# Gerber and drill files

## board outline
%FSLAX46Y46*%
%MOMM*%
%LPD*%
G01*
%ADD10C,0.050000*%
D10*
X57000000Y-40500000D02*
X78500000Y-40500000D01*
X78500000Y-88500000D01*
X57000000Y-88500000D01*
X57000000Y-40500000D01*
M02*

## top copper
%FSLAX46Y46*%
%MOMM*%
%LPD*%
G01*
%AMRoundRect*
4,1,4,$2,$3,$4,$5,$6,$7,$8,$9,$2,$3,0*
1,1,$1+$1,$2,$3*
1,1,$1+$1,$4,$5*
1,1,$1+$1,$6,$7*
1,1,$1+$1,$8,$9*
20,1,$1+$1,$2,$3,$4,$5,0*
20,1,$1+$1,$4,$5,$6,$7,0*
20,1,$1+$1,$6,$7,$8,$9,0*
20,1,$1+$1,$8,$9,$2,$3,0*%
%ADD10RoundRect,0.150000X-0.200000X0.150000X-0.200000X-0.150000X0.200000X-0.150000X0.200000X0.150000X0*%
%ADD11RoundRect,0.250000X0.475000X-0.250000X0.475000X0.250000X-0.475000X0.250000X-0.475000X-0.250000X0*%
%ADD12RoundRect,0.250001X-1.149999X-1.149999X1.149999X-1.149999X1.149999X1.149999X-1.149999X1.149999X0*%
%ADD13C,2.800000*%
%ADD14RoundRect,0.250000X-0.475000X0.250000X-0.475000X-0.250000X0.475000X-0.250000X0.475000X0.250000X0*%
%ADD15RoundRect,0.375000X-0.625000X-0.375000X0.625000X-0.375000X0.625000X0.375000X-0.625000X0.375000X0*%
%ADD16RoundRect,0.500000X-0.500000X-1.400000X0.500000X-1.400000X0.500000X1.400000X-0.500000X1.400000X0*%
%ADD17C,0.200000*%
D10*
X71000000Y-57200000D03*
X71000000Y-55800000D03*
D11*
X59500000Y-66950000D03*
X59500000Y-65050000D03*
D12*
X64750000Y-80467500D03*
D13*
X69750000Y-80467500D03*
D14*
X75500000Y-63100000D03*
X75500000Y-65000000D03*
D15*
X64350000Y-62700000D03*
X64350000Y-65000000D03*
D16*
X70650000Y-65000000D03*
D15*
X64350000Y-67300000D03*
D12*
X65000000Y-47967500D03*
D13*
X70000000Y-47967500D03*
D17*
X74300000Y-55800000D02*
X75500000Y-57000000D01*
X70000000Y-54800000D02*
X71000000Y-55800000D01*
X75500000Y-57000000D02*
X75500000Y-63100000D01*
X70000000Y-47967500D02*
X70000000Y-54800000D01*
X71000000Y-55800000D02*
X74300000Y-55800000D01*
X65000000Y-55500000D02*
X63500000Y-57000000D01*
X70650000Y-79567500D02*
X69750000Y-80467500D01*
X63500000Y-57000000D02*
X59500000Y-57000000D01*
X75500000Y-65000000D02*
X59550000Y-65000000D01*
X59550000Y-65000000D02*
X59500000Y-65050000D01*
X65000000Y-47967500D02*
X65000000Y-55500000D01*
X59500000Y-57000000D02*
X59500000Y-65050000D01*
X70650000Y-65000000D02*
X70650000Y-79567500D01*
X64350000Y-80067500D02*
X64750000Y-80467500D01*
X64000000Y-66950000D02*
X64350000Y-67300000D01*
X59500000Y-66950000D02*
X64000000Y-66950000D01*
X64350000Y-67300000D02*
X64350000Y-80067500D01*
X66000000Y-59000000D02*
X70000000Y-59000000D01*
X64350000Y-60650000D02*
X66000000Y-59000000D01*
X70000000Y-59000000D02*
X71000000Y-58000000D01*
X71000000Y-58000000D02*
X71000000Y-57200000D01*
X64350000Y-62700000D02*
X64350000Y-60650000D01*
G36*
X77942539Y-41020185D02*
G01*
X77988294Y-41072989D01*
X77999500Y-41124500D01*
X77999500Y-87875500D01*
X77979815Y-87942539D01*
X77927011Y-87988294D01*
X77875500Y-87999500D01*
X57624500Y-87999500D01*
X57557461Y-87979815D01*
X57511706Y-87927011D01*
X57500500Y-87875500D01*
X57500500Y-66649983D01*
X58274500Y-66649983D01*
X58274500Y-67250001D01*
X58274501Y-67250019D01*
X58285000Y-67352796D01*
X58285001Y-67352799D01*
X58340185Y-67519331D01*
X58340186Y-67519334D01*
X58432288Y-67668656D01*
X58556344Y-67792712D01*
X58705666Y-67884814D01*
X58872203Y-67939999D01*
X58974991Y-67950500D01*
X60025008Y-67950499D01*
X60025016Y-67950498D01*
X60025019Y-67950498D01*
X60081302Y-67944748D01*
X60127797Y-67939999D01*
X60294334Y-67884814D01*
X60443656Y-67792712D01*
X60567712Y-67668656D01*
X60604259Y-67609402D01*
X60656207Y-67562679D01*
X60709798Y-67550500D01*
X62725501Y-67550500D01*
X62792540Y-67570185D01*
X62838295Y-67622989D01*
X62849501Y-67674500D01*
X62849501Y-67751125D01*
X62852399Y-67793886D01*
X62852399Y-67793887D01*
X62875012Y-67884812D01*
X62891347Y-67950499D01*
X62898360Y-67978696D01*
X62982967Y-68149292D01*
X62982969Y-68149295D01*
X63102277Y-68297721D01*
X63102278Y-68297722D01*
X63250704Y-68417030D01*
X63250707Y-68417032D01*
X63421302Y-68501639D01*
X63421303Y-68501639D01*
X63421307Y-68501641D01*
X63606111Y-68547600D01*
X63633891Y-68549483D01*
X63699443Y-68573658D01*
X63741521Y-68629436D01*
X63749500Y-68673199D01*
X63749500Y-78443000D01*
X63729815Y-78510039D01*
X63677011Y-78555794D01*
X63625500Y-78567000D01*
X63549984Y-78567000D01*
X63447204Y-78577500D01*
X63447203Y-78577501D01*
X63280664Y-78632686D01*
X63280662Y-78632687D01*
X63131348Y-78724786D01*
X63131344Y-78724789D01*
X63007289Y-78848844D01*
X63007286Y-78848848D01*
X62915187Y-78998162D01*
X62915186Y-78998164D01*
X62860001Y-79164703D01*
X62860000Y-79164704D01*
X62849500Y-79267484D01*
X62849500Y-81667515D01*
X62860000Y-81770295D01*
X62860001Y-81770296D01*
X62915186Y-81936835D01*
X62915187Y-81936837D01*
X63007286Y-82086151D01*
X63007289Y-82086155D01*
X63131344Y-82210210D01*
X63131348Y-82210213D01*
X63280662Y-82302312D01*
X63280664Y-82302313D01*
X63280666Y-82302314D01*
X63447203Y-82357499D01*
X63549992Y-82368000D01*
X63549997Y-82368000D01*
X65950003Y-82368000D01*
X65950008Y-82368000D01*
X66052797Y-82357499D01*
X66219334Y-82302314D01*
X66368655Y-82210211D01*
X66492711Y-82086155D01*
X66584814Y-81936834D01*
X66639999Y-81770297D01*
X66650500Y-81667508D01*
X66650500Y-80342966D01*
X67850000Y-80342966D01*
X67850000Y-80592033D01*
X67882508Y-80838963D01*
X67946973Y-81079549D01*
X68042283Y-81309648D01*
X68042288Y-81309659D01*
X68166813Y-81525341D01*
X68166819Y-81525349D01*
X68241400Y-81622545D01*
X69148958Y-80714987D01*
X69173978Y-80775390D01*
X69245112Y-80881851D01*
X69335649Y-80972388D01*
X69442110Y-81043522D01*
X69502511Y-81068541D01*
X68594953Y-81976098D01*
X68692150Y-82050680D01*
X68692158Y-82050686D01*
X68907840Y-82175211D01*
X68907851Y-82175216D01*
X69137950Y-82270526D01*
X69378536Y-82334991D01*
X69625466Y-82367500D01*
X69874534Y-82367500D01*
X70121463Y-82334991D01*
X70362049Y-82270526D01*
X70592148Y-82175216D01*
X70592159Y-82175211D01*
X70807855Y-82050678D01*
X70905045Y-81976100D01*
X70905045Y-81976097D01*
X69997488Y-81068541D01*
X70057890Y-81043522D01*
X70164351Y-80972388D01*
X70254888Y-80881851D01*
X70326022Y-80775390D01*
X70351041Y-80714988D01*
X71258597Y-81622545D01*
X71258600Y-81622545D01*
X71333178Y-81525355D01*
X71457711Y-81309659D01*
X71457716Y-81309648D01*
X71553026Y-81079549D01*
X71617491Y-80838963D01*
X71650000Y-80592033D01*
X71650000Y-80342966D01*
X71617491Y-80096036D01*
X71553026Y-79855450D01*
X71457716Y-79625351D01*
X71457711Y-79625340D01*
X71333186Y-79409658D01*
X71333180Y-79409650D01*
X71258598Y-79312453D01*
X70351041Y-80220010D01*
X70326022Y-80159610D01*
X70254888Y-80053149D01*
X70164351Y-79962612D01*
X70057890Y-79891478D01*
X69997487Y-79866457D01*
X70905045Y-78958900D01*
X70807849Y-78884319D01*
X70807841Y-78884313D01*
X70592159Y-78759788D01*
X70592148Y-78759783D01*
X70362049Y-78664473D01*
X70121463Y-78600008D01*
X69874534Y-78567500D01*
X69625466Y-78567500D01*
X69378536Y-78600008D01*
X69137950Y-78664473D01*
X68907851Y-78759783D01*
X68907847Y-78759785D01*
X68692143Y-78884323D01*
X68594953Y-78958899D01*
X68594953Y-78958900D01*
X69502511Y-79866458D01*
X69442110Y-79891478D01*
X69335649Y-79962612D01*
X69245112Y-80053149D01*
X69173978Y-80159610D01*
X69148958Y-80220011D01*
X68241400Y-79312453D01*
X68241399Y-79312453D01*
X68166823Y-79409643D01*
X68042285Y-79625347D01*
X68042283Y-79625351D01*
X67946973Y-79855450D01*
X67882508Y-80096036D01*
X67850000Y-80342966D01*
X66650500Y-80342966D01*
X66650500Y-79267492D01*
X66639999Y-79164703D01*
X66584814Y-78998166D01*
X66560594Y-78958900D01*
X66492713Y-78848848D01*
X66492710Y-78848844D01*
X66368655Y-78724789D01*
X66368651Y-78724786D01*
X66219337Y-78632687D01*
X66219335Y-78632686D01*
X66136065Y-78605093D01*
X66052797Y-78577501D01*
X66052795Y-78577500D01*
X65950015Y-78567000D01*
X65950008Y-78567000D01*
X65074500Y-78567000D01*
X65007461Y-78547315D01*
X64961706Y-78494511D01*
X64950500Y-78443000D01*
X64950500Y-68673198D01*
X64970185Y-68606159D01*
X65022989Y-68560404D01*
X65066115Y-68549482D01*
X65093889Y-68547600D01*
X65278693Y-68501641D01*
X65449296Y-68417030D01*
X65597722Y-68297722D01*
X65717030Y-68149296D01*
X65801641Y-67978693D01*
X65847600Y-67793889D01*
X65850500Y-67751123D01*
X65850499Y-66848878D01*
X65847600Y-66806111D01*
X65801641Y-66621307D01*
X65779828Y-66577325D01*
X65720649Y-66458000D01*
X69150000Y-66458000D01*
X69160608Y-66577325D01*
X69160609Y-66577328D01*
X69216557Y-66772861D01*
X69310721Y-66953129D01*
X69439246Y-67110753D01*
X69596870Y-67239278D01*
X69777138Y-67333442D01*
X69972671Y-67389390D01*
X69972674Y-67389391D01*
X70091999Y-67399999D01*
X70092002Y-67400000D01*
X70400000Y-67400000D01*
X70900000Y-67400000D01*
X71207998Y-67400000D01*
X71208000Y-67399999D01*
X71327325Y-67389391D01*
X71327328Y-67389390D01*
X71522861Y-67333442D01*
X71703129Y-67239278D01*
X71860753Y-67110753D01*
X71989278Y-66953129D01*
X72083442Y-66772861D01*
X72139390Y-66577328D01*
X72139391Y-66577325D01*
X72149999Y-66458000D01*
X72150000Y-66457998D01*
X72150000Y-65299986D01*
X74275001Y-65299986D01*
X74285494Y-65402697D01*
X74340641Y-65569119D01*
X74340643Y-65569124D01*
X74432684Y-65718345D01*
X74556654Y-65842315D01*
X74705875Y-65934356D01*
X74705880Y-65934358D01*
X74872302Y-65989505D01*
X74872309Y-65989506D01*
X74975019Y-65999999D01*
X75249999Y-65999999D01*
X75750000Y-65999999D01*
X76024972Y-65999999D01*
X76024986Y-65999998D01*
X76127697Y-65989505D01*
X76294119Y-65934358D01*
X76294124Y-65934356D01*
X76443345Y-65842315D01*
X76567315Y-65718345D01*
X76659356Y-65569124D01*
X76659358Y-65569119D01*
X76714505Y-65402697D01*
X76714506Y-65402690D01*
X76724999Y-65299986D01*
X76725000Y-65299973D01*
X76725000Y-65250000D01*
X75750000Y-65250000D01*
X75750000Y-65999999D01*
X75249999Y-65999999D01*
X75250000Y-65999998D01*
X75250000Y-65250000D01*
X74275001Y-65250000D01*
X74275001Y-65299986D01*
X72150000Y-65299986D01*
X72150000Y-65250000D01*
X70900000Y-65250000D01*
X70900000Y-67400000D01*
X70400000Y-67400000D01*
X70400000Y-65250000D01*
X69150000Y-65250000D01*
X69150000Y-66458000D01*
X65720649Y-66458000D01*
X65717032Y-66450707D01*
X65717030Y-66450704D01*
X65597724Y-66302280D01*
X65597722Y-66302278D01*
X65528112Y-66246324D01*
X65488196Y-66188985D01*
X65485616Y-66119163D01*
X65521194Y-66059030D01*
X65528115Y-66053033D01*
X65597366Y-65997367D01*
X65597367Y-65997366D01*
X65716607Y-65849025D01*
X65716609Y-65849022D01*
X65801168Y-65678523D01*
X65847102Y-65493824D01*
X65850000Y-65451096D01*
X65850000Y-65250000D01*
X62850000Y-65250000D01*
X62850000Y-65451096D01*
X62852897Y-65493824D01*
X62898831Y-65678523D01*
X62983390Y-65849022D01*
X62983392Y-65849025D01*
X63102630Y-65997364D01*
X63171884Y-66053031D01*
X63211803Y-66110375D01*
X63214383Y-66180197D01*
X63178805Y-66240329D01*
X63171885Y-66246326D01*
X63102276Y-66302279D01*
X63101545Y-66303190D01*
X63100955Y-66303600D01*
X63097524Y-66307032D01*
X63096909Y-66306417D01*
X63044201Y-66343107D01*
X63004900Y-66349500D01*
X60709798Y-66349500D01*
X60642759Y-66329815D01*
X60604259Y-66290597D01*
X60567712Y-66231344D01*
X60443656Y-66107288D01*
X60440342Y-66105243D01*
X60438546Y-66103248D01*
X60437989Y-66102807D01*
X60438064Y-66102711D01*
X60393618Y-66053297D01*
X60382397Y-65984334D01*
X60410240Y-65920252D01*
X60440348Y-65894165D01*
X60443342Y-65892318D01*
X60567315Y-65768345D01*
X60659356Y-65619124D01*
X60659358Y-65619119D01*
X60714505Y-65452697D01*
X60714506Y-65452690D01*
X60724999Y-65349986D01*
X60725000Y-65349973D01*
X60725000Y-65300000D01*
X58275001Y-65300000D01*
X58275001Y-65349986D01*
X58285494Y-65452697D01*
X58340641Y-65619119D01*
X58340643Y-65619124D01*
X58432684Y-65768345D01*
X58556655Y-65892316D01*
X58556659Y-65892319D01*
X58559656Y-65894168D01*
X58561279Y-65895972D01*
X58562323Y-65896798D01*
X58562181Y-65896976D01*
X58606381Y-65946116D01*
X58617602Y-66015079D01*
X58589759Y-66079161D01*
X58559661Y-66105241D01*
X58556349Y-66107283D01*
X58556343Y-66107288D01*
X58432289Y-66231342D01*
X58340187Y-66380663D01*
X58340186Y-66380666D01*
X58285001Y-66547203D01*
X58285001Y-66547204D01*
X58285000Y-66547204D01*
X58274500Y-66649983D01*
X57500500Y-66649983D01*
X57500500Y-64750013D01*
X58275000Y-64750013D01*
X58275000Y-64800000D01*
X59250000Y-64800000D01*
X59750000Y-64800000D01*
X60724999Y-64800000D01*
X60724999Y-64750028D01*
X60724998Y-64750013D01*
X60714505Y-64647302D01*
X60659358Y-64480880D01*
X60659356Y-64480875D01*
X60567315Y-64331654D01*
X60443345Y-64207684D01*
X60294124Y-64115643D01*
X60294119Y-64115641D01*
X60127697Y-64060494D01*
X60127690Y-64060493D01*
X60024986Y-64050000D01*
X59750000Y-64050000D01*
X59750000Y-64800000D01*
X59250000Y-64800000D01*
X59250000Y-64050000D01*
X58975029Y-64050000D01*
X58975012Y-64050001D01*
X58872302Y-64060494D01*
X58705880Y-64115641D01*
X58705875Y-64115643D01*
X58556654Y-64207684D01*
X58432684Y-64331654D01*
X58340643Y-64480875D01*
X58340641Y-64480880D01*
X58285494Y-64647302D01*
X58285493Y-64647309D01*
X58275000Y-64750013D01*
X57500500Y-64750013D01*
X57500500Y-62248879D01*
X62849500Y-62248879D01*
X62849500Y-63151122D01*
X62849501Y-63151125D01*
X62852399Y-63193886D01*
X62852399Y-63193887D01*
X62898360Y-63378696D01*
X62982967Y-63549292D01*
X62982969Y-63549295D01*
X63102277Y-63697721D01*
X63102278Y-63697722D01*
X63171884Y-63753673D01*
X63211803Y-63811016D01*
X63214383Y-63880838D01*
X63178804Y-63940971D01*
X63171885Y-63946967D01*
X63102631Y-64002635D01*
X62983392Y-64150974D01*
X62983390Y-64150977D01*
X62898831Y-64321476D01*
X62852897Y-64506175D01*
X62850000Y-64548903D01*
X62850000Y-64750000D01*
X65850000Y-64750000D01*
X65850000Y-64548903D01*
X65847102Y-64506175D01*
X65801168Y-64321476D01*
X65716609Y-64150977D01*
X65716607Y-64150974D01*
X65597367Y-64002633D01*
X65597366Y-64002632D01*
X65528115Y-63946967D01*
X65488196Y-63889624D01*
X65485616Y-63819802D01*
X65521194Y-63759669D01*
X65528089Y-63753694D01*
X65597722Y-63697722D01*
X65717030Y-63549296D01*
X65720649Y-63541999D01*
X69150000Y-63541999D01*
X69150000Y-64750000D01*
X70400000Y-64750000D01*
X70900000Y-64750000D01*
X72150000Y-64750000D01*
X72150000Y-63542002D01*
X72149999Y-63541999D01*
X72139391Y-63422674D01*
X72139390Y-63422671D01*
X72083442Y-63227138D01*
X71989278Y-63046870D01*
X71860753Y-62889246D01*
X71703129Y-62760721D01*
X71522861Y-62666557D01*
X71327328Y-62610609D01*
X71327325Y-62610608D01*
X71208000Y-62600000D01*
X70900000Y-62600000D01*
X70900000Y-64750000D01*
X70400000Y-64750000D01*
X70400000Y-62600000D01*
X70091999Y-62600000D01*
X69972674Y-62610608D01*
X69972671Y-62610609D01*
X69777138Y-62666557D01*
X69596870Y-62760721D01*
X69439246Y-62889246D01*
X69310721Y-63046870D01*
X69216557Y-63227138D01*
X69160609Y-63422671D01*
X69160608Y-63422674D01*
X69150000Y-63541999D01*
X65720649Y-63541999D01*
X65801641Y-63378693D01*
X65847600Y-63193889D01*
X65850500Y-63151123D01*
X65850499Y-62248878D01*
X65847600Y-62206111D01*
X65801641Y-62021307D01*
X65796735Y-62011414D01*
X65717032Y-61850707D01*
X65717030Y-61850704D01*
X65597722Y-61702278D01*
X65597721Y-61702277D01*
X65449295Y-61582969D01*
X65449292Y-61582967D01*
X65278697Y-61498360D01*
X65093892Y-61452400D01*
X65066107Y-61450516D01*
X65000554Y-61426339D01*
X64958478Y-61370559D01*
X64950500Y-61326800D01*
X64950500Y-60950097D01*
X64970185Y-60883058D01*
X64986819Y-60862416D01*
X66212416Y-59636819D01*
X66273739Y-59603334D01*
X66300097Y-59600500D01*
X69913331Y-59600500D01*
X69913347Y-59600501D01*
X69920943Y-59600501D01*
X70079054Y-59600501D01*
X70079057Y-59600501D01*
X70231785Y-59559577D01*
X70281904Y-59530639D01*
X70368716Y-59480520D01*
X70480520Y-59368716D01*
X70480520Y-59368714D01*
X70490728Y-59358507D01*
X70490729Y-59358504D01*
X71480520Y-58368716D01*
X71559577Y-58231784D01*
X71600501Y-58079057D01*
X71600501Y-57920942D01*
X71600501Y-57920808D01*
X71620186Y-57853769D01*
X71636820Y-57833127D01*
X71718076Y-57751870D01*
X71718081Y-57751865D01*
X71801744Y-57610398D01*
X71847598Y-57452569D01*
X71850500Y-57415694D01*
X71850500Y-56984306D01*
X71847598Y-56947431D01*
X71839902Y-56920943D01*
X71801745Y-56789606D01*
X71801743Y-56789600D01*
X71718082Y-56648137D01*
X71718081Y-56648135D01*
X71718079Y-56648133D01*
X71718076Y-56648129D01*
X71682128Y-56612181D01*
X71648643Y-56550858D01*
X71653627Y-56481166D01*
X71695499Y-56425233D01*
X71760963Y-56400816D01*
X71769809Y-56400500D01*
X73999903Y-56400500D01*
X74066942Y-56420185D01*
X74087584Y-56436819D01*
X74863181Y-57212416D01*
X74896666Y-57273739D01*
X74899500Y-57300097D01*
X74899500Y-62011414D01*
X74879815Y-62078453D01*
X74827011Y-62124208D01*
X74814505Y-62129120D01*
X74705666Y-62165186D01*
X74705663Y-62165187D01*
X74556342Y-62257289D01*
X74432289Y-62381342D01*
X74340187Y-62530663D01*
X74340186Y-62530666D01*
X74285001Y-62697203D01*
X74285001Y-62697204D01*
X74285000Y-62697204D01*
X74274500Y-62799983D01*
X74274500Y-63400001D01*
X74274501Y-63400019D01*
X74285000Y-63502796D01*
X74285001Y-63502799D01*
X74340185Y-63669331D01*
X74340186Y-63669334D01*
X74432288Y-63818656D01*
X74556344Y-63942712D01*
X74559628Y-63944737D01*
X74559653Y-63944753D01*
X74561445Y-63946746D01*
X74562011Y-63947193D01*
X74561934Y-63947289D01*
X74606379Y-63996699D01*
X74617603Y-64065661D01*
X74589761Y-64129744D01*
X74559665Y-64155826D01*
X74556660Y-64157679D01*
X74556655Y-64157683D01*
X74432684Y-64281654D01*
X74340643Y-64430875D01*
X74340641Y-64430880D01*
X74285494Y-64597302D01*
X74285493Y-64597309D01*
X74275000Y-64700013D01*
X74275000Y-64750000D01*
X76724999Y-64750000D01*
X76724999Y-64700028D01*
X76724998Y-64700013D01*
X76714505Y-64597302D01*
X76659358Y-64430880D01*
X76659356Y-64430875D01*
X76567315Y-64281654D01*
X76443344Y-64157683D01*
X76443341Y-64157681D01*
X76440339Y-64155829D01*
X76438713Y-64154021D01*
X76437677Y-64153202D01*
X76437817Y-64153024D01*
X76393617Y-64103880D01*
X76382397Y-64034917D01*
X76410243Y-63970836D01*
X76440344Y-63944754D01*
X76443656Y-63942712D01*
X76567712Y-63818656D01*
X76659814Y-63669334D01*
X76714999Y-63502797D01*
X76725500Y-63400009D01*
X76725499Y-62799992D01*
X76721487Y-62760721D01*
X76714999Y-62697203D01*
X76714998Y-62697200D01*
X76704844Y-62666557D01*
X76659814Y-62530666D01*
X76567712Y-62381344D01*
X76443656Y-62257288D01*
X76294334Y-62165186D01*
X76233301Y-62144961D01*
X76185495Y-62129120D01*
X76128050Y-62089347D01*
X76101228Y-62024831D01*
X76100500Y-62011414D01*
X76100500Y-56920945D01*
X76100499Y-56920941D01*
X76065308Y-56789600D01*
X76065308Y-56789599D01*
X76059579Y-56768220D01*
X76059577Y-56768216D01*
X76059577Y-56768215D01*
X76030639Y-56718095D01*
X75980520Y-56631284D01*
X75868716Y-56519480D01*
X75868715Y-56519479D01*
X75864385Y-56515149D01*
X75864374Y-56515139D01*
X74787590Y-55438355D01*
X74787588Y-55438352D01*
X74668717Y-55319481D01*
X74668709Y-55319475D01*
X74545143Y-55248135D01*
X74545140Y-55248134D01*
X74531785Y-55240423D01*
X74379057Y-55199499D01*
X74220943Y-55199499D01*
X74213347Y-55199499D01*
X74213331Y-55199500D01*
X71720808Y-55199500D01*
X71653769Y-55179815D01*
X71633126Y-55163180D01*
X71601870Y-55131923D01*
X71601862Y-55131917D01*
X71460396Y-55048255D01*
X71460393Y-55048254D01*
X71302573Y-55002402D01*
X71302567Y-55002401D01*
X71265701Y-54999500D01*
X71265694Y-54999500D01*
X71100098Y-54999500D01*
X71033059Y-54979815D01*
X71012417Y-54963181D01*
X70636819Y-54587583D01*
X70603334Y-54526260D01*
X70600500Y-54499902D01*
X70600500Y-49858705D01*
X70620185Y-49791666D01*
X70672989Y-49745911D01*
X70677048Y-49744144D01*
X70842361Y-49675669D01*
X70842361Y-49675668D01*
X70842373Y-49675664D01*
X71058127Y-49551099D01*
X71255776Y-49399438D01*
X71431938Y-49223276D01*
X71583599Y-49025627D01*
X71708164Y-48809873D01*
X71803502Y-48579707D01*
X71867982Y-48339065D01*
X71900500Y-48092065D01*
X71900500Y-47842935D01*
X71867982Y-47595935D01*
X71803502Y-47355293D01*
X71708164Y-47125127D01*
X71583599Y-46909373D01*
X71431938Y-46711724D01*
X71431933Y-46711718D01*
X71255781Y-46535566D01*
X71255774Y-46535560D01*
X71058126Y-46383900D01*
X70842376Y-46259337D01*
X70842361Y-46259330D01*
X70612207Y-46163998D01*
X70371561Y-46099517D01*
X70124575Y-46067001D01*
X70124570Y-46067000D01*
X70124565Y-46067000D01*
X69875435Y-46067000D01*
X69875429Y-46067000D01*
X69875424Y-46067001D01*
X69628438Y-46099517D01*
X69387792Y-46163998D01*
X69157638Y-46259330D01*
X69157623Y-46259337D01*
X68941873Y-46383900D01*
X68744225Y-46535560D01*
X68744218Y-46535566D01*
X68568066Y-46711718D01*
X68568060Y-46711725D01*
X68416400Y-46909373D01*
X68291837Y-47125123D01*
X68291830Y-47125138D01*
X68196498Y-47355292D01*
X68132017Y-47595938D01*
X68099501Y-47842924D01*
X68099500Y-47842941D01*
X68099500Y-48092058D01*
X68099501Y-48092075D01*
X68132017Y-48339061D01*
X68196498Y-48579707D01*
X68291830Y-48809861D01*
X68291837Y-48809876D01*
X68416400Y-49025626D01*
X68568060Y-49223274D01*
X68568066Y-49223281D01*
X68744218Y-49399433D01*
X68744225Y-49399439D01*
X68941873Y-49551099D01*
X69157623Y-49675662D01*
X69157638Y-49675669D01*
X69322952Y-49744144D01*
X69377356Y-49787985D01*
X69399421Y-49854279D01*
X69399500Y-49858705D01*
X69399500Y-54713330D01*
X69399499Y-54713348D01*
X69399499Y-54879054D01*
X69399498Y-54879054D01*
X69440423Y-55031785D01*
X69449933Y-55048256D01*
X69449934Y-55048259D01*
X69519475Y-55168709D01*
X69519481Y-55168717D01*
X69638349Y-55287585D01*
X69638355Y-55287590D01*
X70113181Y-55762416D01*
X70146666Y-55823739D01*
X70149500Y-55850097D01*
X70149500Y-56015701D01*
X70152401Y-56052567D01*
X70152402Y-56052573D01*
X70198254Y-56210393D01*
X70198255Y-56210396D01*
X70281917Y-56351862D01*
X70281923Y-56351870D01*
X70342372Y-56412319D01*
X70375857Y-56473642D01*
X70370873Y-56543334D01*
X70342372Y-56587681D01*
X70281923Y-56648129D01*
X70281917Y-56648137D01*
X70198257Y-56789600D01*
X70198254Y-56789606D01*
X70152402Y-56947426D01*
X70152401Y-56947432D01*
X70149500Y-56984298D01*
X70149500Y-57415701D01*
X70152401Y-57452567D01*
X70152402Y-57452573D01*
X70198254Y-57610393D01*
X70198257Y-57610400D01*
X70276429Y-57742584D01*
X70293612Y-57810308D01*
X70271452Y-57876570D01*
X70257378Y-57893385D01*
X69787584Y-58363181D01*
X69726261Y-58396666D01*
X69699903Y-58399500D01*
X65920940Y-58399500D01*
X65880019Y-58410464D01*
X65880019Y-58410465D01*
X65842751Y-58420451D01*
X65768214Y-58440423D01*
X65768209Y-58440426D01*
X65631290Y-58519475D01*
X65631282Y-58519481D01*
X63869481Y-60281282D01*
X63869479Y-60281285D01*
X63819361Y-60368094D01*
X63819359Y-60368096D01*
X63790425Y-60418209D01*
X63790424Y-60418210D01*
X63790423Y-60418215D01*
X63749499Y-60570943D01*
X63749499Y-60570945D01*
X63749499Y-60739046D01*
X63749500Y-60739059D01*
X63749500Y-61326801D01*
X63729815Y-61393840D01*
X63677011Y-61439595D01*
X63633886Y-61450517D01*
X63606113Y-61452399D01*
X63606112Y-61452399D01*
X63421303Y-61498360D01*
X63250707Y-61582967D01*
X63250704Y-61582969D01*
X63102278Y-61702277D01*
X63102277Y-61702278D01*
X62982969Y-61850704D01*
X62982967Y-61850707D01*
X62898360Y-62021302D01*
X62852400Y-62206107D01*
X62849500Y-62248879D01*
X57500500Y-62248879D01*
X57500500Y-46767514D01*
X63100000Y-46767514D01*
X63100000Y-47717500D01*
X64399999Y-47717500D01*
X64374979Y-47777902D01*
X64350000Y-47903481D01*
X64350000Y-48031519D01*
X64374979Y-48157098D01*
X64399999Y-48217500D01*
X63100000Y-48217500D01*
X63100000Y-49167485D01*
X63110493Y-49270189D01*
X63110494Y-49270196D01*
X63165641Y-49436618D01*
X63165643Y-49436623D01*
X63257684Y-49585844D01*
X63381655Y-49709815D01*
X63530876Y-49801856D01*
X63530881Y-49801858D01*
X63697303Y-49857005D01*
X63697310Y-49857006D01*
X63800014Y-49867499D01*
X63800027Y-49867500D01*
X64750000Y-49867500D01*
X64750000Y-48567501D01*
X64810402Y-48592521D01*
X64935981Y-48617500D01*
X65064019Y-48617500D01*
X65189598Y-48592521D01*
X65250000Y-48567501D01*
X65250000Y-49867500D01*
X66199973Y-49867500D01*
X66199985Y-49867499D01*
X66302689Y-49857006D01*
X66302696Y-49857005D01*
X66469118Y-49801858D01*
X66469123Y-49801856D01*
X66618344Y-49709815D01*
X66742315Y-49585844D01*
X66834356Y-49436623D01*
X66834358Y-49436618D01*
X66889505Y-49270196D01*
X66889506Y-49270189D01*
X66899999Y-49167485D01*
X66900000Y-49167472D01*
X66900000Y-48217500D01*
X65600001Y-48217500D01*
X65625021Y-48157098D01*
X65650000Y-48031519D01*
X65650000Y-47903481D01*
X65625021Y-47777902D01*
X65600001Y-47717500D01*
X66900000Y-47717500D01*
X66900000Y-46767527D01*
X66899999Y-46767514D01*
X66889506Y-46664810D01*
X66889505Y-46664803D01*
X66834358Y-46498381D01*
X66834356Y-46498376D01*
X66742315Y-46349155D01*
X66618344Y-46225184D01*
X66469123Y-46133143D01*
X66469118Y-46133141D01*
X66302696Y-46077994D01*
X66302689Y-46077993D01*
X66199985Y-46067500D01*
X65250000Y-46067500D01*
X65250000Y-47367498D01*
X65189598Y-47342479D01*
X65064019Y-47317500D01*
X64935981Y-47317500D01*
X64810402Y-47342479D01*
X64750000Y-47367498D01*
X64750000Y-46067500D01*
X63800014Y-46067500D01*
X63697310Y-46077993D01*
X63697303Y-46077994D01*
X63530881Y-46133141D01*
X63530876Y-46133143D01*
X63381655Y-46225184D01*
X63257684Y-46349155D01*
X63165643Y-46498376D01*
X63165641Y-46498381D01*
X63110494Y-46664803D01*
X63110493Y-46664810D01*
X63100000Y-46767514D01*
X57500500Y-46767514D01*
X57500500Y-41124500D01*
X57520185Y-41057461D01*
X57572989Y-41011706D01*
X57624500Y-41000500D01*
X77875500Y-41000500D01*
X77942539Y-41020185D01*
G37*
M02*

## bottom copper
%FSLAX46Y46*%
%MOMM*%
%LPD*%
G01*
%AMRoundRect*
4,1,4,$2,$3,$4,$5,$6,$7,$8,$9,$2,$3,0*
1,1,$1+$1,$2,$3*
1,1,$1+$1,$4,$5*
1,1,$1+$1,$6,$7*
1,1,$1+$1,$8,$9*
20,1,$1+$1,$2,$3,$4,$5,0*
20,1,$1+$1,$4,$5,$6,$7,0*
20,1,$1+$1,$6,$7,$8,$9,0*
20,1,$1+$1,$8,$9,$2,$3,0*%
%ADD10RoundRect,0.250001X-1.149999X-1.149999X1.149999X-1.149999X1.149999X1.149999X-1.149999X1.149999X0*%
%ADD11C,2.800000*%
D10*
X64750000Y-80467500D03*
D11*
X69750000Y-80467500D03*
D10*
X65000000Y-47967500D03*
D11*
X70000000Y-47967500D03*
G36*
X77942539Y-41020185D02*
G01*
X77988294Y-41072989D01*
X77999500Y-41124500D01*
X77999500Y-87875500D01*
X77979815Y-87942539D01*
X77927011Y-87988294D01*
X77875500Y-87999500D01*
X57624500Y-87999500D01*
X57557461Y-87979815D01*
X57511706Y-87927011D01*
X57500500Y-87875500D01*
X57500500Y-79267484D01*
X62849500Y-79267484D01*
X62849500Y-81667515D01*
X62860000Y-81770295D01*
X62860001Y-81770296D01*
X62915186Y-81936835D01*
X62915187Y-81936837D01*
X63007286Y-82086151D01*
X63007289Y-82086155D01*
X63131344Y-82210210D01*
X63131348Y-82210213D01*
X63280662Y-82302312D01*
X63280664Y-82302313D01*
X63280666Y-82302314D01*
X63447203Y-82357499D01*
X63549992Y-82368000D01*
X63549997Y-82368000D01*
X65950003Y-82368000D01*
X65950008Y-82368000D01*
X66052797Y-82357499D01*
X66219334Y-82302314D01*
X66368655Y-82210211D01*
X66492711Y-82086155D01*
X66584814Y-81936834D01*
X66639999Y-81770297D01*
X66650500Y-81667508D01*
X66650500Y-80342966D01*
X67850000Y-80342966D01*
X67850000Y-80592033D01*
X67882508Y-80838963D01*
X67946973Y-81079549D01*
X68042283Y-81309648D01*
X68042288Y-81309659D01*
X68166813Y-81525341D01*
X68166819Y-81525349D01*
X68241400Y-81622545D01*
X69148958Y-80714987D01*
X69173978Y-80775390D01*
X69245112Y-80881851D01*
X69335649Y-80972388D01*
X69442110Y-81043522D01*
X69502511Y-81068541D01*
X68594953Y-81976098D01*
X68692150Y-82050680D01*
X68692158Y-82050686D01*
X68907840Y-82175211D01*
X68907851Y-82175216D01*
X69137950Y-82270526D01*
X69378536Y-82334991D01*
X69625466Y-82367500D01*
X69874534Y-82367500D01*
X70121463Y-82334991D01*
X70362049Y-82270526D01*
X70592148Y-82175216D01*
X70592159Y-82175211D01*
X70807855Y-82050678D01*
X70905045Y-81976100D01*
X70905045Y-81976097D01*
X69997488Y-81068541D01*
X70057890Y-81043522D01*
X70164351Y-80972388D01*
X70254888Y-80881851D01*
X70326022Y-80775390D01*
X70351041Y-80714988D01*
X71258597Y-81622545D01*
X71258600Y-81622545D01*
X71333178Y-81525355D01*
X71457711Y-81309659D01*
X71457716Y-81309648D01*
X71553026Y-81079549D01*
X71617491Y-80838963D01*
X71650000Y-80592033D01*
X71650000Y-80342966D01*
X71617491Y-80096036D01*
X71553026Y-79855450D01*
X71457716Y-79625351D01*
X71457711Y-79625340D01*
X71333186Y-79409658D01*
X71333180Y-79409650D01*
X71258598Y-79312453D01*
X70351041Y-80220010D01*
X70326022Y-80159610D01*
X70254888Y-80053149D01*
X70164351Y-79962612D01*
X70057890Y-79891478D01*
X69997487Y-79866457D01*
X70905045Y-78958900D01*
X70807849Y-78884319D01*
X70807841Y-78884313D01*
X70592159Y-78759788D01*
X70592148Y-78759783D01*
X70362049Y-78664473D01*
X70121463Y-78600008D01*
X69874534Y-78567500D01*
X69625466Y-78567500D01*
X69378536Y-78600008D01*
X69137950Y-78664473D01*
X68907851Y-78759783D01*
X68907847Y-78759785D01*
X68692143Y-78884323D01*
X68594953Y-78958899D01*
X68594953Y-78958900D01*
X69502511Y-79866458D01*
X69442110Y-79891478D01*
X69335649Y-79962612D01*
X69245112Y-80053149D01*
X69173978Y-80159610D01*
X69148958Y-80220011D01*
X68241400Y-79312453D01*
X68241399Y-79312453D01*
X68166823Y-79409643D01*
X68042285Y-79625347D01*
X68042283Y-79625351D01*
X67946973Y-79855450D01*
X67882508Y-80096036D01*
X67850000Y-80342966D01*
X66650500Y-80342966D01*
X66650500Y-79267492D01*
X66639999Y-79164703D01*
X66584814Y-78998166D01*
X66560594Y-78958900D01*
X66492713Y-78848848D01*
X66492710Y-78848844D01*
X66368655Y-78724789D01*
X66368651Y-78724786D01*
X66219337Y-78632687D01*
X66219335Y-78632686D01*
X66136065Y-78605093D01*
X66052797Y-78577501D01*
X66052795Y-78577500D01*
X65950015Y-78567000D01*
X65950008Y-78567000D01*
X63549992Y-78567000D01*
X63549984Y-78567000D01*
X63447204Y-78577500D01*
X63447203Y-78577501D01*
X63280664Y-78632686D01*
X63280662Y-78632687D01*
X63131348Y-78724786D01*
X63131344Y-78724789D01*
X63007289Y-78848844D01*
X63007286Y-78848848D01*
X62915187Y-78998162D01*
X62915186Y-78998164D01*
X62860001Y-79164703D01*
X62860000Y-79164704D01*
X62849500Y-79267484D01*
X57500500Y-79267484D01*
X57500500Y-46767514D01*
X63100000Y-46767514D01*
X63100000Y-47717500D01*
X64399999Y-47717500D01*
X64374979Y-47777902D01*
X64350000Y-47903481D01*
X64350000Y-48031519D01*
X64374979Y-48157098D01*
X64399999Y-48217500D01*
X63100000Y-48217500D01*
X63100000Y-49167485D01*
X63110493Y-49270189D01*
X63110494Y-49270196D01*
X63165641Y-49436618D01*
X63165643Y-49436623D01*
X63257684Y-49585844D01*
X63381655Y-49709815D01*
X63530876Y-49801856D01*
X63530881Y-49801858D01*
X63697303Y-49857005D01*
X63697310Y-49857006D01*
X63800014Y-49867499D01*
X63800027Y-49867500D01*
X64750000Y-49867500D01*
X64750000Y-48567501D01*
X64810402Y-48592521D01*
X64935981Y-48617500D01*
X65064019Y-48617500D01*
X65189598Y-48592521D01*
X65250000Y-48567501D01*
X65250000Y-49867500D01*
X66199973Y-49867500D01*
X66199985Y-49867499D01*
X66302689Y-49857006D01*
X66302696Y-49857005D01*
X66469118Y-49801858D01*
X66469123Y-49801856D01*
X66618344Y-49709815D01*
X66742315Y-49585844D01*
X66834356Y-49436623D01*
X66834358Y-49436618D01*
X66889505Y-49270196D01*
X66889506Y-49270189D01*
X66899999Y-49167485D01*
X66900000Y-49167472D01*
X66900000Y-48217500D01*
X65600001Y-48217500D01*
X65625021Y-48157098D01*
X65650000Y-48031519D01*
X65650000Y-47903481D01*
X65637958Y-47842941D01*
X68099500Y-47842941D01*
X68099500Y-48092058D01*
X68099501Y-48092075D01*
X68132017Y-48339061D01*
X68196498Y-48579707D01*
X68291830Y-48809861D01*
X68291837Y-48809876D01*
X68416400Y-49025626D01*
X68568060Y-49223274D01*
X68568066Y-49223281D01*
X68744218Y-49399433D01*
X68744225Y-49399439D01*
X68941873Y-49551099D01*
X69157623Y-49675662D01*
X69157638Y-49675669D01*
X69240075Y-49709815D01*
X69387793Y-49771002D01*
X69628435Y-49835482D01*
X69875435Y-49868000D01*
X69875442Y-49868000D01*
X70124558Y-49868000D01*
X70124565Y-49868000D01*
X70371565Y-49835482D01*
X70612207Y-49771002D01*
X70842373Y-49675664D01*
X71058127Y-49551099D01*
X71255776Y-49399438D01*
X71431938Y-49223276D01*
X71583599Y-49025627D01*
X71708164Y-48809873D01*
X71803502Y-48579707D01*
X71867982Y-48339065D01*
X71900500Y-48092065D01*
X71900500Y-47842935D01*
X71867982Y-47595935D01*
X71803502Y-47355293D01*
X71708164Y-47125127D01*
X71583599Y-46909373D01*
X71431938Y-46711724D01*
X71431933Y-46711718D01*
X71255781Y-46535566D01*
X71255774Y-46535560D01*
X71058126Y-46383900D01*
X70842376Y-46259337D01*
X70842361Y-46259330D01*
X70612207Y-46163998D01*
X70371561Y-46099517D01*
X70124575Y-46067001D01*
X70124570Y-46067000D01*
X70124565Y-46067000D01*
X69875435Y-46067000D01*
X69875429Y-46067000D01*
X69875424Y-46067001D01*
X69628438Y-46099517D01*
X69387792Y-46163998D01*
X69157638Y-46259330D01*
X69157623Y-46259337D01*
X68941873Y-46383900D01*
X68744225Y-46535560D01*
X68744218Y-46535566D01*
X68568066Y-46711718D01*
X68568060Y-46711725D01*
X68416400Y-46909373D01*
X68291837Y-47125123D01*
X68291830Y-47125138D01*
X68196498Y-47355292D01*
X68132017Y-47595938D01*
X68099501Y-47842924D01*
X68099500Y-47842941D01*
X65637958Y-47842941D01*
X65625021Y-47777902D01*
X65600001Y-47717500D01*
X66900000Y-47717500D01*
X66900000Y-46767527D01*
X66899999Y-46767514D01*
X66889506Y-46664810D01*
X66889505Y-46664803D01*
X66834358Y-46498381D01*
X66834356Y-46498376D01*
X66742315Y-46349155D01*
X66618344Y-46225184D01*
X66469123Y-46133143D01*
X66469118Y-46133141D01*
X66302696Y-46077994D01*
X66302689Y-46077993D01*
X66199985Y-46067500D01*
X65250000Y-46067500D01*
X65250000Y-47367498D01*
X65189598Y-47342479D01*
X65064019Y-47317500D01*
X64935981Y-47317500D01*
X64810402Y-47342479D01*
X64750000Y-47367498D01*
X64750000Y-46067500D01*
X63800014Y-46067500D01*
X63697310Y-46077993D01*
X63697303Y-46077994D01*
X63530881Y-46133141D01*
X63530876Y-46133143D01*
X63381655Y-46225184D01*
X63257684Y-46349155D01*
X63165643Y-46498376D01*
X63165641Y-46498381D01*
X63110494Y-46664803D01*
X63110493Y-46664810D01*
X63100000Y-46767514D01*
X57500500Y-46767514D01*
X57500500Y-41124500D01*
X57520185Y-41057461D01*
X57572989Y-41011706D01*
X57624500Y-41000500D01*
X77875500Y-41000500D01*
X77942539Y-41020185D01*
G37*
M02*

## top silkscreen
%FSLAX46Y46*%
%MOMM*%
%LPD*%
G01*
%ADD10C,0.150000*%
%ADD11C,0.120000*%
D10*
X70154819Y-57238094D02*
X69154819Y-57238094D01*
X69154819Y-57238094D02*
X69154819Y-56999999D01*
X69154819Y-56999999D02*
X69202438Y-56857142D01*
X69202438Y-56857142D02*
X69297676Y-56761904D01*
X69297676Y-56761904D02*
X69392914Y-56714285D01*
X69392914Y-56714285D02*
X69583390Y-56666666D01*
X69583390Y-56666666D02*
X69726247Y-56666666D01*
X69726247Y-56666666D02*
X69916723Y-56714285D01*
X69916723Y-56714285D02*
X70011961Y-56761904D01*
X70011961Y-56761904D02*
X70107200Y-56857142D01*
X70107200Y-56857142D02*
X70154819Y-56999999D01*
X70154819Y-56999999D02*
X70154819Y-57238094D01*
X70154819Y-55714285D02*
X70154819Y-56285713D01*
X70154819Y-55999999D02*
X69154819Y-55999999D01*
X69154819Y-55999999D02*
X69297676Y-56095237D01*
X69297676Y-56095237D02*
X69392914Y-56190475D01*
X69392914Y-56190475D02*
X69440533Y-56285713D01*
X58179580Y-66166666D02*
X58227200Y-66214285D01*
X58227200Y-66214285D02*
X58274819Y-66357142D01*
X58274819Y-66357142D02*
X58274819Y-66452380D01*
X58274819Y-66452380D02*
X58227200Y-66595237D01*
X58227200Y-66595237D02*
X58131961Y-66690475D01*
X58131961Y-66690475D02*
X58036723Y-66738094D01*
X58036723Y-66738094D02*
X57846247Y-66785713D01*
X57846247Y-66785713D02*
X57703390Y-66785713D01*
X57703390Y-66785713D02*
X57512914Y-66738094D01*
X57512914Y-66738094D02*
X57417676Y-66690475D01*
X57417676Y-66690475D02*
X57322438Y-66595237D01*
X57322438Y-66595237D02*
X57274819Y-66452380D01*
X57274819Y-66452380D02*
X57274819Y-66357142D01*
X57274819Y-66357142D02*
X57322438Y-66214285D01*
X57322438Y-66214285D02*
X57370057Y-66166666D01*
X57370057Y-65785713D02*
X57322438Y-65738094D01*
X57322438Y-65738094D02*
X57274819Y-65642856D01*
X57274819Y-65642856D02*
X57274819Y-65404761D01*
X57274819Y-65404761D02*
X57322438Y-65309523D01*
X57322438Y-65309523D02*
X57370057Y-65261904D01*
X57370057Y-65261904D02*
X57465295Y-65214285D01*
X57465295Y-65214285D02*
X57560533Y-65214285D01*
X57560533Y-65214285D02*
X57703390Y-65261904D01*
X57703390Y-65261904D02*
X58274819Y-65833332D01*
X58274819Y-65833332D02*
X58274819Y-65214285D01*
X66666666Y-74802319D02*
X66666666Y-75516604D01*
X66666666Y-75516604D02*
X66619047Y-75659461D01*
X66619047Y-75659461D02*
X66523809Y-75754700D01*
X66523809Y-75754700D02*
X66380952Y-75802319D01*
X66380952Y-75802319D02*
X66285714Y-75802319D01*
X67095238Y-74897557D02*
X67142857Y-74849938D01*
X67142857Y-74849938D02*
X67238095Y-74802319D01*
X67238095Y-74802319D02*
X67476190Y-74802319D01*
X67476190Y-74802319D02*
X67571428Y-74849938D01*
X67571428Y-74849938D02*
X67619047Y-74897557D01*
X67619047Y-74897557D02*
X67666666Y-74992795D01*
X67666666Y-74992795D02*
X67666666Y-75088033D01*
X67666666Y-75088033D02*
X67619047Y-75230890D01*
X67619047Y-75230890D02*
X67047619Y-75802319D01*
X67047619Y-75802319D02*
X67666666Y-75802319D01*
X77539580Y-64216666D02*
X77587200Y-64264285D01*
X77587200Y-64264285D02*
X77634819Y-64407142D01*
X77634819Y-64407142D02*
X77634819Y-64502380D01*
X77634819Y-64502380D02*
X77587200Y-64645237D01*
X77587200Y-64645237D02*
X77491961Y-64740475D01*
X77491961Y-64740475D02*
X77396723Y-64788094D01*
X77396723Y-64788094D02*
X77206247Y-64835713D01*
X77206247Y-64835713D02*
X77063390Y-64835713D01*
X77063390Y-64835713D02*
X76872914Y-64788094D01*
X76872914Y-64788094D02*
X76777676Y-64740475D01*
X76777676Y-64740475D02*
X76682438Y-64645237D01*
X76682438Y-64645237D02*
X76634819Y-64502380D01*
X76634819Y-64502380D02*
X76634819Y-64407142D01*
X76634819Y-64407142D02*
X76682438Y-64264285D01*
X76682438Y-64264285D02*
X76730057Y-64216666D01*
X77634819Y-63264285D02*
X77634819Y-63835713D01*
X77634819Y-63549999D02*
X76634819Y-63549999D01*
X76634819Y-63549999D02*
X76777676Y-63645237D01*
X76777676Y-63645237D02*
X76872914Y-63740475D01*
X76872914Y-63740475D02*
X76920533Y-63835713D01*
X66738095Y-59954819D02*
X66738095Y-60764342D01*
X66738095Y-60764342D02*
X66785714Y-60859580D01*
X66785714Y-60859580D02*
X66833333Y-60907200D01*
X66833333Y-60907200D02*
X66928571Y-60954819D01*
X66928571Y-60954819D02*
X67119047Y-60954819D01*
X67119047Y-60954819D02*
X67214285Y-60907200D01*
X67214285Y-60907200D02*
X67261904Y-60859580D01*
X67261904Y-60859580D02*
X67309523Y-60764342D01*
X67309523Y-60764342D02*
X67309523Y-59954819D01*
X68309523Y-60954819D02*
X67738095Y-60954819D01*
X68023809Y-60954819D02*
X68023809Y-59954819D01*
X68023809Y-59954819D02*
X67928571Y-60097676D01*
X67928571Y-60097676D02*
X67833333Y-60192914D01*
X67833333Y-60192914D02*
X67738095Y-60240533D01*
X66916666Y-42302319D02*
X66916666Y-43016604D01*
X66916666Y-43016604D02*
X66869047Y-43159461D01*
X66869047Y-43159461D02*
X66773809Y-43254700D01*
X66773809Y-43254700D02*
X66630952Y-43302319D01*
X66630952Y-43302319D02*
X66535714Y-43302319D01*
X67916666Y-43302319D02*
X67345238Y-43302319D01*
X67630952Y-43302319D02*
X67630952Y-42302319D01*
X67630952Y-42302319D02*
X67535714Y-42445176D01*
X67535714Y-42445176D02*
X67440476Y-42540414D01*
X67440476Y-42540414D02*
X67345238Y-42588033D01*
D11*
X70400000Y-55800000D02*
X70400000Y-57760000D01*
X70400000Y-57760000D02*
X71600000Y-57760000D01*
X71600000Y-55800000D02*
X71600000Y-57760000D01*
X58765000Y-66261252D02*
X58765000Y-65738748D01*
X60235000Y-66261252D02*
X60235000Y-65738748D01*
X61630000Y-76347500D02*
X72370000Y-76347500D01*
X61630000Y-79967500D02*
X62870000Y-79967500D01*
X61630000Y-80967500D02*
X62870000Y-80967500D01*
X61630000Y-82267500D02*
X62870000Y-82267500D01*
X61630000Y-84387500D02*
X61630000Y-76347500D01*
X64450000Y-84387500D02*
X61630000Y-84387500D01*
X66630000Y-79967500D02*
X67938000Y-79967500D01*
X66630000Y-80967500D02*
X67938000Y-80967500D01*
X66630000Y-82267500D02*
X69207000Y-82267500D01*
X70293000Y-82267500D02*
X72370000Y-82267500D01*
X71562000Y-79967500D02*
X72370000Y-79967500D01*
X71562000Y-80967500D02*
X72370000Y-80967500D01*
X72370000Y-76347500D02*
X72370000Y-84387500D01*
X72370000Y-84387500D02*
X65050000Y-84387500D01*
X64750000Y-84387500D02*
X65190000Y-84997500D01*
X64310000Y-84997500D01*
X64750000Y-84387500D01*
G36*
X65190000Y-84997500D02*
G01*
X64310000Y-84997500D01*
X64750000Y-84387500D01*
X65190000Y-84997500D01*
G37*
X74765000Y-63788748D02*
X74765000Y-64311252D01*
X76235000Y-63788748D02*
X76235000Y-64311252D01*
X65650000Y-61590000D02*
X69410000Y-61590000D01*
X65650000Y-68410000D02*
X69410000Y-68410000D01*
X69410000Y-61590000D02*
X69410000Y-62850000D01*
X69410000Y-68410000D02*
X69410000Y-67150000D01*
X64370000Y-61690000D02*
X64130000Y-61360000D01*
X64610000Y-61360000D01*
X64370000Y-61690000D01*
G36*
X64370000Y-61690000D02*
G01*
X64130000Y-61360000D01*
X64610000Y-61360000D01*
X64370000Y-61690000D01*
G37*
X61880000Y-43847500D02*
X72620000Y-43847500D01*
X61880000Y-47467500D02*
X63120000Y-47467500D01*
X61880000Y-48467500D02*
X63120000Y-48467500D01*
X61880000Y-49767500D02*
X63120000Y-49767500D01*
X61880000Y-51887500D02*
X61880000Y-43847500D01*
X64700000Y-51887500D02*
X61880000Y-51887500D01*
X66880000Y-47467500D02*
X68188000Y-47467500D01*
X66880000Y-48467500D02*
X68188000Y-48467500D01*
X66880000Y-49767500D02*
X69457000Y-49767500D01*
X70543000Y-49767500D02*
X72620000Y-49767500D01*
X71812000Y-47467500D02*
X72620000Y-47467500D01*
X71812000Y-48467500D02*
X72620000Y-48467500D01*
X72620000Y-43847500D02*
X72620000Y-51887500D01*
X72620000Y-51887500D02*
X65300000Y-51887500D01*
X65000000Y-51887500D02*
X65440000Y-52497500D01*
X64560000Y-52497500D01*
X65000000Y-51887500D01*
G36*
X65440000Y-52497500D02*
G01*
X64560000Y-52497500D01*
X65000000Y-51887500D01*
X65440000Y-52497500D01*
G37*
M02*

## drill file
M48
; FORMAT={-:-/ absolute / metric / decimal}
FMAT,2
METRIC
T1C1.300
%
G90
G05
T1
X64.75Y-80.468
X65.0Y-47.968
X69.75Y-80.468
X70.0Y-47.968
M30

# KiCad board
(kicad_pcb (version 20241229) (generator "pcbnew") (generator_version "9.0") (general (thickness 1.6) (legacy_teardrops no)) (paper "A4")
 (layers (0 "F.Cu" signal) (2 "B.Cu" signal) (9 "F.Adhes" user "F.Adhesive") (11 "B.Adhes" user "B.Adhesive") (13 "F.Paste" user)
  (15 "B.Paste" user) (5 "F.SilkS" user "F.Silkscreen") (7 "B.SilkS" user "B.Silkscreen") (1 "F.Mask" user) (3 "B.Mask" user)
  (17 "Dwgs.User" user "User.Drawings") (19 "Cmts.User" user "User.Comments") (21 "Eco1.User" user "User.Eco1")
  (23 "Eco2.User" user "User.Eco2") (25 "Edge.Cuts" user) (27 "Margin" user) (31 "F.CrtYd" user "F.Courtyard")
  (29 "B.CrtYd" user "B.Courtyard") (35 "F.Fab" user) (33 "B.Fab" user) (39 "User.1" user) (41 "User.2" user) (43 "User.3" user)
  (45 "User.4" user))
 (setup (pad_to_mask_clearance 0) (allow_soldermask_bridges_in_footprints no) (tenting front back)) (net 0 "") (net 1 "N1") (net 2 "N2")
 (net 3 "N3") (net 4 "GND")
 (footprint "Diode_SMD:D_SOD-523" (layer "F.Cu") (at 71 56.5 90)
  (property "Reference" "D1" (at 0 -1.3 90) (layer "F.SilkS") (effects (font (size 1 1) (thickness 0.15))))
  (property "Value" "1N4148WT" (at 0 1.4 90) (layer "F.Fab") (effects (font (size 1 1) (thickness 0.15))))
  (fp_line (start 0.7 -0.6) (end -1.26 -0.6) (stroke (width 0.12) (type solid)) (layer "F.SilkS"))
  (fp_line (start -1.26 -0.6) (end -1.26 0.6) (stroke (width 0.12) (type solid)) (layer "F.SilkS"))
  (fp_line (start 0.7 0.6) (end -1.26 0.6) (stroke (width 0.12) (type solid)) (layer "F.SilkS"))
  (pad "1" smd roundrect (at -0.7 0 270) (size 0.6 0.7) (layers "F.Cu" "F.Mask" "F.Paste") (roundrect_rratio 0.25) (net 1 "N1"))
  (pad "2" smd roundrect (at 0.7 0 270) (size 0.6 0.7) (layers "F.Cu" "F.Mask" "F.Paste") (roundrect_rratio 0.25) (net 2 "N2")))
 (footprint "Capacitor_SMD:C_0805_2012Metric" (layer "F.Cu") (at 59.5 66 90)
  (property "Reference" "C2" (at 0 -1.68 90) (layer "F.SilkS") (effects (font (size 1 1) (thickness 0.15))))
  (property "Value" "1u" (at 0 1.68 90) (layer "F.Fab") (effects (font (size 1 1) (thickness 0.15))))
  (fp_line (start -0.261252 -0.735) (end 0.261252 -0.735) (stroke (width 0.12) (type solid)) (layer "F.SilkS"))
  (fp_line (start -0.261252 0.735) (end 0.261252 0.735) (stroke (width 0.12) (type solid)) (layer "F.SilkS"))
  (pad "1" smd roundrect (at -0.95 0 90) (size 1 1.45) (layers "F.Cu" "F.Mask" "F.Paste") (roundrect_rratio 0.25) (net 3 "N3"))
  (pad "2" smd roundrect (at 0.95 0 90) (size 1 1.45) (layers "F.Cu" "F.Mask" "F.Paste") (roundrect_rratio 0.25) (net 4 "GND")))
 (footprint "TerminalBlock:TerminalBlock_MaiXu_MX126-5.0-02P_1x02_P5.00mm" (layer "F.Cu") (at 64.75 80.4675)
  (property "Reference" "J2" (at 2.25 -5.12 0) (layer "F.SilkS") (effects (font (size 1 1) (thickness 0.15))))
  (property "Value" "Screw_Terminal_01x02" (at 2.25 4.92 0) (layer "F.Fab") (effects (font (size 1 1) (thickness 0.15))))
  (fp_line (start -3.12 -4.12) (end 7.62 -4.12) (stroke (width 0.12) (type solid)) (layer "F.SilkS"))
  (fp_line (start -3.12 -0.5) (end -1.88 -0.5) (stroke (width 0.12) (type solid)) (layer "F.SilkS"))
  (fp_line (start -3.12 0.5) (end -1.88 0.5) (stroke (width 0.12) (type solid)) (layer "F.SilkS"))
  (fp_line (start -3.12 1.8) (end -1.88 1.8) (stroke (width 0.12) (type solid)) (layer "F.SilkS"))
  (fp_line (start -3.12 3.92) (end -3.12 -4.12) (stroke (width 0.12) (type solid)) (layer "F.SilkS"))
  (fp_line (start -0.3 3.92) (end -3.12 3.92) (stroke (width 0.12) (type solid)) (layer "F.SilkS"))
  (fp_line (start 1.88 -0.5) (end 3.188 -0.5) (stroke (width 0.12) (type solid)) (layer "F.SilkS"))
  (fp_line (start 1.88 0.5) (end 3.188 0.5) (stroke (width 0.12) (type solid)) (layer "F.SilkS"))
  (fp_line (start 1.88 1.8) (end 4.457 1.8) (stroke (width 0.12) (type solid)) (layer "F.SilkS"))
  (fp_line (start 5.543 1.8) (end 7.62 1.8) (stroke (width 0.12) (type solid)) (layer "F.SilkS"))
  (fp_line (start 6.812 -0.5) (end 7.62 -0.5) (stroke (width 0.12) (type solid)) (layer "F.SilkS"))
  (fp_line (start 6.812 0.5) (end 7.62 0.5) (stroke (width 0.12) (type solid)) (layer "F.SilkS"))
  (fp_line (start 7.62 -4.12) (end 7.62 3.92) (stroke (width 0.12) (type solid)) (layer "F.SilkS"))
  (fp_line (start 7.62 3.92) (end 0.3 3.92) (stroke (width 0.12) (type solid)) (layer "F.SilkS"))
  (fp_poly (pts (xy 0 3.92) (xy 0.44 4.53) (xy -0.44 4.53)) (stroke (width 0.12) (type solid)) (fill yes) (layer "F.SilkS"))
  (pad "1" thru_hole roundrect (at 0 0) (size 2.8 2.8) (drill 1.3) (layers "*.Cu" "*.Mask") (remove_unused_layers no)
   (roundrect_rratio 0.089286) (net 3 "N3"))
  (pad "2" thru_hole circle (at 5 0) (size 2.8 2.8) (drill 1.3) (layers "*.Cu" "*.Mask") (remove_unused_layers no) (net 4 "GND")))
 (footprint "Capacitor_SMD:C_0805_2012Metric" (layer "F.Cu") (at 75.5 64.05 -90)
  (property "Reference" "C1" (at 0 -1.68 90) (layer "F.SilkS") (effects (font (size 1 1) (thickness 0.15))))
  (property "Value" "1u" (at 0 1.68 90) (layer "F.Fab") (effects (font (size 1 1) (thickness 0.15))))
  (fp_line (start -0.261252 0.735) (end 0.261252 0.735) (stroke (width 0.12) (type solid)) (layer "F.SilkS"))
  (fp_line (start -0.261252 -0.735) (end 0.261252 -0.735) (stroke (width 0.12) (type solid)) (layer "F.SilkS"))
  (pad "1" smd roundrect (at -0.95 0 270) (size 1 1.45) (layers "F.Cu" "F.Mask" "F.Paste") (roundrect_rratio 0.25) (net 2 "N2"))
  (pad "2" smd roundrect (at 0.95 0 270) (size 1 1.45) (layers "F.Cu" "F.Mask" "F.Paste") (roundrect_rratio 0.25) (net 4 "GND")))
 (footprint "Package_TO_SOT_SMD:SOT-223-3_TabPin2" (layer "F.Cu") (at 67.5 65)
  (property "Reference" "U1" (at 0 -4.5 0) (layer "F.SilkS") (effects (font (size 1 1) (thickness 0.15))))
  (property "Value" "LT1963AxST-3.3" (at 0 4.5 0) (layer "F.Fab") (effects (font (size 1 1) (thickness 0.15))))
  (fp_line (start -1.85 -3.41) (end 1.91 -3.41) (stroke (width 0.12) (type solid)) (layer "F.SilkS"))
  (fp_line (start -1.85 3.41) (end 1.91 3.41) (stroke (width 0.12) (type solid)) (layer "F.SilkS"))
  (fp_line (start 1.91 -3.41) (end 1.91 -2.15) (stroke (width 0.12) (type solid)) (layer "F.SilkS"))
  (fp_line (start 1.91 3.41) (end 1.91 2.15) (stroke (width 0.12) (type solid)) (layer "F.SilkS"))
  (fp_poly
   (pts (xy -3.13 -3.31) (xy -3.37 -3.64) (xy -2.89 -3.64) (xy -3.13 -3.31)) (stroke (width 0.12) (type solid)) (fill yes) (layer "F.SilkS"))
  (pad "1" smd roundrect (at -3.15 -2.3) (size 2 1.5) (layers "F.Cu" "F.Mask" "F.Paste") (roundrect_rratio 0.25) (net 1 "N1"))
  (pad "2" smd roundrect (at -3.15 0) (size 2 1.5) (layers "F.Cu" "F.Mask" "F.Paste") (roundrect_rratio 0.25) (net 4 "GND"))
  (pad "2" smd roundrect (at 3.15 0) (size 2 3.8) (layers "F.Cu" "F.Mask" "F.Paste") (roundrect_rratio 0.25) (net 4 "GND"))
  (pad "3" smd roundrect (at -3.15 2.3) (size 2 1.5) (layers "F.Cu" "F.Mask" "F.Paste") (roundrect_rratio 0.25) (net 3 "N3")))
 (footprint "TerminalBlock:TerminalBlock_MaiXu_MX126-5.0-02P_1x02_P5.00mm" (layer "F.Cu") (at 65 47.9675)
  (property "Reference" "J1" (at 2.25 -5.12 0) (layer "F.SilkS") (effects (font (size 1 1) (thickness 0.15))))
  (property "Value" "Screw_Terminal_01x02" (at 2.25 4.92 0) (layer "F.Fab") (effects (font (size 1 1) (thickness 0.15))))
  (fp_line (start -3.12 -4.12) (end 7.62 -4.12) (stroke (width 0.12) (type solid)) (layer "F.SilkS"))
  (fp_line (start -3.12 -0.5) (end -1.88 -0.5) (stroke (width 0.12) (type solid)) (layer "F.SilkS"))
  (fp_line (start -3.12 0.5) (end -1.88 0.5) (stroke (width 0.12) (type solid)) (layer "F.SilkS"))
  (fp_line (start -3.12 1.8) (end -1.88 1.8) (stroke (width 0.12) (type solid)) (layer "F.SilkS"))
  (fp_line (start -3.12 3.92) (end -3.12 -4.12) (stroke (width 0.12) (type solid)) (layer "F.SilkS"))
  (fp_line (start -0.3 3.92) (end -3.12 3.92) (stroke (width 0.12) (type solid)) (layer "F.SilkS"))
  (fp_line (start 1.88 -0.5) (end 3.188 -0.5) (stroke (width 0.12) (type solid)) (layer "F.SilkS"))
  (fp_line (start 1.88 0.5) (end 3.188 0.5) (stroke (width 0.12) (type solid)) (layer "F.SilkS"))
  (fp_line (start 1.88 1.8) (end 4.457 1.8) (stroke (width 0.12) (type solid)) (layer "F.SilkS"))
  (fp_line (start 5.543 1.8) (end 7.62 1.8) (stroke (width 0.12) (type solid)) (layer "F.SilkS"))
  (fp_line (start 6.812 -0.5) (end 7.62 -0.5) (stroke (width 0.12) (type solid)) (layer "F.SilkS"))
  (fp_line (start 6.812 0.5) (end 7.62 0.5) (stroke (width 0.12) (type solid)) (layer "F.SilkS"))
  (fp_line (start 7.62 -4.12) (end 7.62 3.92) (stroke (width 0.12) (type solid)) (layer "F.SilkS"))
  (fp_line (start 7.62 3.92) (end 0.3 3.92) (stroke (width 0.12) (type solid)) (layer "F.SilkS"))
  (fp_poly (pts (xy 0 3.92) (xy 0.44 4.53) (xy -0.44 4.53)) (stroke (width 0.12) (type solid)) (fill yes) (layer "F.SilkS"))
  (pad "1" thru_hole roundrect (at 0 0) (size 2.8 2.8) (drill 1.3) (layers "*.Cu" "*.Mask") (remove_unused_layers no)
   (roundrect_rratio 0.089286) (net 4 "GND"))
  (pad "2" thru_hole circle (at 5 0) (size 2.8 2.8) (drill 1.3) (layers "*.Cu" "*.Mask") (remove_unused_layers no) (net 2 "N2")))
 (gr_rect (start 57 40.5) (end 78.5 88.5) (stroke (width 0.05) (type default)) (fill no) (layer "Edge.Cuts"))
 (segment (start 74.3 55.8) (end 75.5 57) (width 0.2) (layer "F.Cu") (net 2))
 (segment (start 70 54.8) (end 71 55.8) (width 0.2) (layer "F.Cu") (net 2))
 (segment (start 75.5 57) (end 75.5 63.1) (width 0.2) (layer "F.Cu") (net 2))
 (segment (start 70 47.9675) (end 70 54.8) (width 0.2) (layer "F.Cu") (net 2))
 (segment (start 71 55.8) (end 74.3 55.8) (width 0.2) (layer "F.Cu") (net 2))
 (segment (start 65 55.5) (end 63.5 57) (width 0.2) (layer "F.Cu") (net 4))
 (segment (start 70.65 79.5675) (end 69.75 80.4675) (width 0.2) (layer "F.Cu") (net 4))
 (segment (start 63.5 57) (end 59.5 57) (width 0.2) (layer "F.Cu") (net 4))
 (segment (start 75.5 65) (end 59.55 65) (width 0.2) (layer "F.Cu") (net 4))
 (segment (start 59.55 65) (end 59.5 65.05) (width 0.2) (layer "F.Cu") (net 4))
 (segment (start 65 47.9675) (end 65 55.5) (width 0.2) (layer "F.Cu") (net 4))
 (segment (start 59.5 57) (end 59.5 65.05) (width 0.2) (layer "F.Cu") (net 4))
 (segment (start 70.65 65) (end 70.65 79.5675) (width 0.2) (layer "F.Cu") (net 4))
 (segment (start 64.35 80.0675) (end 64.75 80.4675) (width 0.2) (layer "F.Cu") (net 3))
 (segment (start 64 66.95) (end 64.35 67.3) (width 0.2) (layer "F.Cu") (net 3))
 (segment (start 59.5 66.95) (end 64 66.95) (width 0.2) (layer "F.Cu") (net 3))
 (segment (start 64.35 67.3) (end 64.35 80.0675) (width 0.2) (layer "F.Cu") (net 3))
 (segment (start 66 59) (end 70 59) (width 0.2) (layer "F.Cu") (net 1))
 (segment (start 64.35 60.65) (end 66 59) (width 0.2) (layer "F.Cu") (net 1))
 (segment (start 70 59) (end 71 58) (width 0.2) (layer "F.Cu") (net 1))
 (segment (start 71 58) (end 71 57.2) (width 0.2) (layer "F.Cu") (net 1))
 (segment (start 64.35 62.7) (end 64.35 60.65) (width 0.2) (layer "F.Cu") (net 1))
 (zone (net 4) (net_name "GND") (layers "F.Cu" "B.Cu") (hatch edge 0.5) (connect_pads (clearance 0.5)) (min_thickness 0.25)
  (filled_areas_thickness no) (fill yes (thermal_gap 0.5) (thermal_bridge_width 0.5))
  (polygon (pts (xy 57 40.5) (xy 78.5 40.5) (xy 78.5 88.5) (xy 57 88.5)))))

